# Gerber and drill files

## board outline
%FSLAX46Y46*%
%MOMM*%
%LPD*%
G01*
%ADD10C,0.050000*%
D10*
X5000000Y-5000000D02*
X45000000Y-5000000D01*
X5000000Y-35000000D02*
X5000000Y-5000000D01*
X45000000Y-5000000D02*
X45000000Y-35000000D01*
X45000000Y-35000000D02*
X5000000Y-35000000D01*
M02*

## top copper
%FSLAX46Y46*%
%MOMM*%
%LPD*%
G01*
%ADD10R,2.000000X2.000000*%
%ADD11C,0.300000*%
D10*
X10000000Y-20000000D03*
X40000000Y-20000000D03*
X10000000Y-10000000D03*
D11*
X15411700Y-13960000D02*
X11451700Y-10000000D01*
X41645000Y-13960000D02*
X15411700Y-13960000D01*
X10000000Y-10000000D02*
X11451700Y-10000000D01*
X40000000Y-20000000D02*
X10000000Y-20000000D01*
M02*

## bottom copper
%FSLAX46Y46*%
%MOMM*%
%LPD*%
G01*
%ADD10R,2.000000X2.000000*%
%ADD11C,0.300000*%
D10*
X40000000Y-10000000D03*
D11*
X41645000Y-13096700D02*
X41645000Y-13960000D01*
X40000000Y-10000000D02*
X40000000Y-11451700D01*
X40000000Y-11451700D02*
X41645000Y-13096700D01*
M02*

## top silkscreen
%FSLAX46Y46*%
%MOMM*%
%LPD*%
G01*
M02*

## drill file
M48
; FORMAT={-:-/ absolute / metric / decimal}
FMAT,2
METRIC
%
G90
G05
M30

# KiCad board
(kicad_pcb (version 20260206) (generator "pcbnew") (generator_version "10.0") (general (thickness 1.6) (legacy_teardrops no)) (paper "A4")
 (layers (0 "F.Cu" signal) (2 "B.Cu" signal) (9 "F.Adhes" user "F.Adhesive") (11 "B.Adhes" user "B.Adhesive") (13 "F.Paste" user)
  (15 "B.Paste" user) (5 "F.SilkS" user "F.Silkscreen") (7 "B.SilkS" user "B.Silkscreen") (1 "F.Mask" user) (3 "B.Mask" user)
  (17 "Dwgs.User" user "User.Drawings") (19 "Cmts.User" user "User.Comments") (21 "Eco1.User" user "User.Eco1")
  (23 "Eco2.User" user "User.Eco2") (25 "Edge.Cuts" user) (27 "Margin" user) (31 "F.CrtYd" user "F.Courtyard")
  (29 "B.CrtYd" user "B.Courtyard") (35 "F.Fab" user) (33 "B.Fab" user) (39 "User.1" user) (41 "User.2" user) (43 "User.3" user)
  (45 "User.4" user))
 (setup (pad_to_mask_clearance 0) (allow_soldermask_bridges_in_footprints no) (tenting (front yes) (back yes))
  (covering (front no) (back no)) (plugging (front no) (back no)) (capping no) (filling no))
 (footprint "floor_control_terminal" (layer "F.Cu") (at 10 20)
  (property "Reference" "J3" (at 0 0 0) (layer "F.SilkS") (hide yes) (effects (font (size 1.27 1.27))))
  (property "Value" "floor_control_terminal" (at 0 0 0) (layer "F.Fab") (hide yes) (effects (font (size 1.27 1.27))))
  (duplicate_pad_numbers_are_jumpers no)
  (pad "1" smd rect (at 0 0) (size 2 2) (layers "F.Cu" "F.Mask" "F.Paste") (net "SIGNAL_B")))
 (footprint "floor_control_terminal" (layer "F.Cu") (at 40 20)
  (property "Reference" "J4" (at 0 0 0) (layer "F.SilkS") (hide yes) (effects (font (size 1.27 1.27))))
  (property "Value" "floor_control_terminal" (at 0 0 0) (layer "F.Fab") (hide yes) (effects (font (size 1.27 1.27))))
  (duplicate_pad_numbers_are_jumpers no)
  (pad "1" smd rect (at 0 0) (size 2 2) (layers "F.Cu" "F.Mask" "F.Paste") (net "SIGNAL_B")))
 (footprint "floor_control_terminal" (layer "F.Cu") (at 10 10)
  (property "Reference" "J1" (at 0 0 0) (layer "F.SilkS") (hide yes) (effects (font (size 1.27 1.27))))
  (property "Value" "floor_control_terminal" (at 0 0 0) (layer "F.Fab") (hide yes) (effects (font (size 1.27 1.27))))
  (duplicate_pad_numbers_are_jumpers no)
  (pad "1" smd rect (at 0 0) (size 2 2) (layers "F.Cu" "F.Mask" "F.Paste") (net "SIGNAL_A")))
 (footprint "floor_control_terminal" (layer "B.Cu") (at 40 10)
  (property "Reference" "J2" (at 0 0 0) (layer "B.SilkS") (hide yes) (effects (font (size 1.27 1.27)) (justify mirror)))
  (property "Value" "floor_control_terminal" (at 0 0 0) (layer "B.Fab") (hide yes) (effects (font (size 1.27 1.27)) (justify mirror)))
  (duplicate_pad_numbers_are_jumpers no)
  (pad "1" smd rect (at 0 0) (size 2 2) (layers "B.Cu" "B.Mask" "B.Paste") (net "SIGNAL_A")))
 (gr_line (start 5 5) (end 45 5) (stroke (width 0.05) (type default)) (layer "Edge.Cuts"))
 (gr_line (start 5 35) (end 5 5) (stroke (width 0.05) (type default)) (layer "Edge.Cuts"))
 (gr_line (start 45 5) (end 45 35) (stroke (width 0.05) (type default)) (layer "Edge.Cuts"))
 (gr_line (start 45 35) (end 5 35) (stroke (width 0.05) (type default)) (layer "Edge.Cuts"))
 (segment (start 15.4117 13.96) (end 11.4517 10) (width 0.3) (layer "F.Cu") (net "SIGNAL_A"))
 (segment (start 41.645 13.96) (end 15.4117 13.96) (width 0.3) (layer "F.Cu") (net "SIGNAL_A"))
 (segment (start 10 10) (end 11.4517 10) (width 0.3) (layer "F.Cu") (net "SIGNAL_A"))
 (segment (start 41.645 13.0967) (end 41.645 13.96) (width 0.3) (layer "B.Cu") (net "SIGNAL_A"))
 (segment (start 40 10) (end 40 11.4517) (width 0.3) (layer "B.Cu") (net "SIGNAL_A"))
 (segment (start 40 11.4517) (end 41.645 13.0967) (width 0.3) (layer "B.Cu") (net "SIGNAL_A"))
 (segment (start 40 20) (end 10 20) (width 0.3) (layer "F.Cu") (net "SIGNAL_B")))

